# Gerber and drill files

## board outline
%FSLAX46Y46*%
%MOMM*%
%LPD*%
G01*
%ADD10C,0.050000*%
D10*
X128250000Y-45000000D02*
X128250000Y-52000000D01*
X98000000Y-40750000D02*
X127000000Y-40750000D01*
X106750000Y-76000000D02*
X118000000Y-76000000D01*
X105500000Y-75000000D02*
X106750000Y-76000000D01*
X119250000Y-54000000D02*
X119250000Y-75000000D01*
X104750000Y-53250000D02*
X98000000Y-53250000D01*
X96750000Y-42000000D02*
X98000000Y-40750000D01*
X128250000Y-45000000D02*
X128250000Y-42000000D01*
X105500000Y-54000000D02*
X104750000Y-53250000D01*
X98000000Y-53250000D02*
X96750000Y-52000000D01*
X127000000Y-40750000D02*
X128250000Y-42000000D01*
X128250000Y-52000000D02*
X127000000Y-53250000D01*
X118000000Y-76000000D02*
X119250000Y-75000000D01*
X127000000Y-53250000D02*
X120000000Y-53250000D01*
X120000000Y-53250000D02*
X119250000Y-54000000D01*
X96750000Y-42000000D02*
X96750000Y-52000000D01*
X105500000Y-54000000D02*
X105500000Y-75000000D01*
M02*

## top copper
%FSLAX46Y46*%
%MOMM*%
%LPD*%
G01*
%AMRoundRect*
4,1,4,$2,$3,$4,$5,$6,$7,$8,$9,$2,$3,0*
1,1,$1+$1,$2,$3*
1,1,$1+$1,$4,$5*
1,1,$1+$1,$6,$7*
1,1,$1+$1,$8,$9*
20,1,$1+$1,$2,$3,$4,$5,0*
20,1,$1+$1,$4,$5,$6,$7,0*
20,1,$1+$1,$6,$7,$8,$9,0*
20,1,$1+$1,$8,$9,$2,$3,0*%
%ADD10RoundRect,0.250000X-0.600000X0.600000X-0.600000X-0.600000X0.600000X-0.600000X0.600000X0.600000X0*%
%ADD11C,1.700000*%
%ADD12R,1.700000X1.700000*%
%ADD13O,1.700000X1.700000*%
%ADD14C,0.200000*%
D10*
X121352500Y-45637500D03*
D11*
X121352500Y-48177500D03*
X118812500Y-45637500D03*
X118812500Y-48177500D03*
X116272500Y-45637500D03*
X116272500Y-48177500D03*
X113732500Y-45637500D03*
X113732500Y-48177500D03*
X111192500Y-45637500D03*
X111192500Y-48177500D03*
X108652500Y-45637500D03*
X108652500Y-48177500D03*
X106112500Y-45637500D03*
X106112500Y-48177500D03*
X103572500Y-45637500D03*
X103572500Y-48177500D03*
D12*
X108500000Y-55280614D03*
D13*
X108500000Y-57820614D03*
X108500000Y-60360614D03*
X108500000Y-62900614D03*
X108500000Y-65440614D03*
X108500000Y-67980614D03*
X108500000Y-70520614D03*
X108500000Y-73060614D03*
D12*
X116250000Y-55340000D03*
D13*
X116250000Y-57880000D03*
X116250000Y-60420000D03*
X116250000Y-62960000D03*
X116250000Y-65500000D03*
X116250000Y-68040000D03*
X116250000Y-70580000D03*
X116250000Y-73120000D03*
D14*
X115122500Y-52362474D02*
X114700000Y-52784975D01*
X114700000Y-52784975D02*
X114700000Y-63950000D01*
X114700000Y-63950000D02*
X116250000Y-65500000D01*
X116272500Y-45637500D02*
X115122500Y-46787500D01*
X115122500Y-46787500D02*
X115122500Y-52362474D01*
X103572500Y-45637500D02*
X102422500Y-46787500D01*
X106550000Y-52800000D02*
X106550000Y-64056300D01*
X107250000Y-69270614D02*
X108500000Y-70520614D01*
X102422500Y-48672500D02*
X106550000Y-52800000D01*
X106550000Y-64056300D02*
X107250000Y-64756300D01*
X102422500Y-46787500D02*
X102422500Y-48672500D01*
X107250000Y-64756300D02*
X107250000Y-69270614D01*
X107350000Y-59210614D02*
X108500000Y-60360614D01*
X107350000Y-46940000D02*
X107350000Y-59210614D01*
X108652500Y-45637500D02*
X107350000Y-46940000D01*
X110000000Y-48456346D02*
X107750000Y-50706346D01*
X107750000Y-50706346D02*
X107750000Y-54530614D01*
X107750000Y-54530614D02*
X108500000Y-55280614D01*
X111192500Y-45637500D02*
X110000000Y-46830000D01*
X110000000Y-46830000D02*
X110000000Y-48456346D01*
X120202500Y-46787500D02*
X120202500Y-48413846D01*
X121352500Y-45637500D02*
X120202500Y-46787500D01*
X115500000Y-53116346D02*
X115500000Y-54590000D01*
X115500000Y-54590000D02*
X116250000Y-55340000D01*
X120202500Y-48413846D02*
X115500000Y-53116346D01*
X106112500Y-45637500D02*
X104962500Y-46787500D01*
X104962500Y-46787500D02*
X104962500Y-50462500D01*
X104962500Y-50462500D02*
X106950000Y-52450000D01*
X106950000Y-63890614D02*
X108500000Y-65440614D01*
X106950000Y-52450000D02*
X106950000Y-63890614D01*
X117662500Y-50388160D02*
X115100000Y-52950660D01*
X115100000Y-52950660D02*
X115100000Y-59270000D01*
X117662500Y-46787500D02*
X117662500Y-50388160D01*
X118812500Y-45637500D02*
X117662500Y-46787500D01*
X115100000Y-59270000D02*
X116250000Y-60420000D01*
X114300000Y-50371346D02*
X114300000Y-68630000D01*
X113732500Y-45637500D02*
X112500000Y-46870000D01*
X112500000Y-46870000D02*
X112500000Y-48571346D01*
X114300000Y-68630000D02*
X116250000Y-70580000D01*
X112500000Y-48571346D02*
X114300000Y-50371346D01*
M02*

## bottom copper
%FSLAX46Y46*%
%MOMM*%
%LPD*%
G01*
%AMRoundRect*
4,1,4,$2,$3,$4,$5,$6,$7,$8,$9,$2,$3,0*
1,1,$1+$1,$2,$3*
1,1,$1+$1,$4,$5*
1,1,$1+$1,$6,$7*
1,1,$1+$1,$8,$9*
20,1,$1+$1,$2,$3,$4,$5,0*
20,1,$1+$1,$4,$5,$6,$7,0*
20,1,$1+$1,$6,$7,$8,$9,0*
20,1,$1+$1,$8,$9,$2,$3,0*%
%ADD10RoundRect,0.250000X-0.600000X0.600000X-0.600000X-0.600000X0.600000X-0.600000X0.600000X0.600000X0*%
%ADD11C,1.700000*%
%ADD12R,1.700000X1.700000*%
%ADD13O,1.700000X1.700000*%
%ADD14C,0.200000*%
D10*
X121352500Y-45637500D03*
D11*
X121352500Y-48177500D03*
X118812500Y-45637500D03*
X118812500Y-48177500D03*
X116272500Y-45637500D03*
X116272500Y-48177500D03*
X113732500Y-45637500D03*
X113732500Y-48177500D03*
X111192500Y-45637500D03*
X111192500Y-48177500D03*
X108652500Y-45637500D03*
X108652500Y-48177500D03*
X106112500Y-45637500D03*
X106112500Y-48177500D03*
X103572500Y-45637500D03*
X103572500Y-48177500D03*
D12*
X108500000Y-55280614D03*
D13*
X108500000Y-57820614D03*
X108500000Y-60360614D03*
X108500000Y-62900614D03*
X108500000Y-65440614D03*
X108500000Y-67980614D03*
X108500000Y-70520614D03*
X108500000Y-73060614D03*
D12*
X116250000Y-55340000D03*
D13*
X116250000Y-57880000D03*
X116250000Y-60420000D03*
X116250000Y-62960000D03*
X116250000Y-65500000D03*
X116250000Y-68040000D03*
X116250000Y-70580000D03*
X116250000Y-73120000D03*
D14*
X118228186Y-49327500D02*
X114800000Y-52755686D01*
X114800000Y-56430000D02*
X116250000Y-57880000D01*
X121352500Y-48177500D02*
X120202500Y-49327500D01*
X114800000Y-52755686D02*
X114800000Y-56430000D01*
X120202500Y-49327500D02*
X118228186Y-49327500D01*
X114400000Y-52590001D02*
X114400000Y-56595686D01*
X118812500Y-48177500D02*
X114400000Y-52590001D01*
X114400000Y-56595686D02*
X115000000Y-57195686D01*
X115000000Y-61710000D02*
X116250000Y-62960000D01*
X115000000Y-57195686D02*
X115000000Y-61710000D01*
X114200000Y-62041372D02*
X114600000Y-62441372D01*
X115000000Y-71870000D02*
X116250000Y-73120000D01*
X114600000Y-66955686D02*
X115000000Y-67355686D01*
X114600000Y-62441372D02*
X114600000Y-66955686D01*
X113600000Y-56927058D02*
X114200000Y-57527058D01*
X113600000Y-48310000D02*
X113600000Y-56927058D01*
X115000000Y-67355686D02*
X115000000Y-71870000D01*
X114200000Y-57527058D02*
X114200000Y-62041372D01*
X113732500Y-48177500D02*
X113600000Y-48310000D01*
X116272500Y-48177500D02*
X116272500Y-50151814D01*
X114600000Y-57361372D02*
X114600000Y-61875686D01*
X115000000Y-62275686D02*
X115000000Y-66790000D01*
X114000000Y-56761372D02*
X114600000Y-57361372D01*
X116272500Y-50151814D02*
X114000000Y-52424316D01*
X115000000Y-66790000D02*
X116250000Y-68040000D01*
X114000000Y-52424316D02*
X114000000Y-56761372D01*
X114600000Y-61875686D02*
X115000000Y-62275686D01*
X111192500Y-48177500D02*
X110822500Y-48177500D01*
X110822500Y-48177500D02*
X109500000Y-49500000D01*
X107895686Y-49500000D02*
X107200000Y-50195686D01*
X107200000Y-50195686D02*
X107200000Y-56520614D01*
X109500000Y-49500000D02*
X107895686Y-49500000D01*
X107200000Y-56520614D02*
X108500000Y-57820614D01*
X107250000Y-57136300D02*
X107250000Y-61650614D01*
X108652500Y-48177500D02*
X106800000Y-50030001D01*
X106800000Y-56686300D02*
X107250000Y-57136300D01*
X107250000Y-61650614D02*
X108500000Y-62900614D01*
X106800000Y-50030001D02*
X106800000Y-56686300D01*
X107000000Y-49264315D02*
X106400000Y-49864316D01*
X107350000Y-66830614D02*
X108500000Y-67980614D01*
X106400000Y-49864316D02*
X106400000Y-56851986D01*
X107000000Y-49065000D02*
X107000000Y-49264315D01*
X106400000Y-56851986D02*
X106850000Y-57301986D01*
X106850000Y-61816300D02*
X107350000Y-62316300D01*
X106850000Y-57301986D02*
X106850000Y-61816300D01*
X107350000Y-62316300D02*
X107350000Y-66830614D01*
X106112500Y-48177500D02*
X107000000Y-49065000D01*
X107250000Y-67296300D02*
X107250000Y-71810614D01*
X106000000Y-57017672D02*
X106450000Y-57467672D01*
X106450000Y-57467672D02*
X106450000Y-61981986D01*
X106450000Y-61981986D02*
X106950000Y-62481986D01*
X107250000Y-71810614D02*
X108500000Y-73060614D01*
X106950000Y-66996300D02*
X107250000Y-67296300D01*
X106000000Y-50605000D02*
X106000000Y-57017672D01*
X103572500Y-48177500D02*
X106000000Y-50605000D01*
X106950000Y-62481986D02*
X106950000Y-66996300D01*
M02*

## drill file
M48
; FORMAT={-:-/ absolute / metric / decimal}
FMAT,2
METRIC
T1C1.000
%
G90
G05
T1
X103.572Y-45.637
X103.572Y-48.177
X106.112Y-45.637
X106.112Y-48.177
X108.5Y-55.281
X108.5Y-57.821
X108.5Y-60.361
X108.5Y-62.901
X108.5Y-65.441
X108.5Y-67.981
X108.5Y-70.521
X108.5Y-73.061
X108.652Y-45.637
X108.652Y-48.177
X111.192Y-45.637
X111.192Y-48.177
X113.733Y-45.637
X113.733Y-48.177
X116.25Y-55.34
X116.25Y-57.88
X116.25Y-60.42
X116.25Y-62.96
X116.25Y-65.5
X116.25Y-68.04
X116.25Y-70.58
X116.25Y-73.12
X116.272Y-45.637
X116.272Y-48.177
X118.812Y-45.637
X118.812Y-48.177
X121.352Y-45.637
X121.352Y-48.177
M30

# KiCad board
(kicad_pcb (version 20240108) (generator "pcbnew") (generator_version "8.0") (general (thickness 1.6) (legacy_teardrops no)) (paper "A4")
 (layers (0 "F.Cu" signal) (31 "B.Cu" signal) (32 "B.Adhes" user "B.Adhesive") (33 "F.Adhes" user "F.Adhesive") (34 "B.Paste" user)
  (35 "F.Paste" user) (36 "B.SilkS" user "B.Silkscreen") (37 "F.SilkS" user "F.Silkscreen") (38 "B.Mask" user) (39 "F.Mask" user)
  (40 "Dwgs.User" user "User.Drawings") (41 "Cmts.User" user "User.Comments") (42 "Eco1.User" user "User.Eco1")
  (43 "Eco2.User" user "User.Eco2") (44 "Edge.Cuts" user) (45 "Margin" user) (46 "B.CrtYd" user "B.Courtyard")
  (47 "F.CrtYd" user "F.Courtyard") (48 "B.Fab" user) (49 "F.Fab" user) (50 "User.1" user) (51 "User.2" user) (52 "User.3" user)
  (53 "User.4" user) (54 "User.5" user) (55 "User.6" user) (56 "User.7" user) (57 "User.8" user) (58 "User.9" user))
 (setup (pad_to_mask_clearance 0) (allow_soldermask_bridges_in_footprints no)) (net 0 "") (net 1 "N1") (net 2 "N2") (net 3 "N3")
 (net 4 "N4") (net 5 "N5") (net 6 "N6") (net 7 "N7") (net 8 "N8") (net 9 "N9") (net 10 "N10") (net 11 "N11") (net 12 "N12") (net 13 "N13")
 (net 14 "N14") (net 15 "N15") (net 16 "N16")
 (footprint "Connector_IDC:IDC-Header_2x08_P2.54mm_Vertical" (layer "F.Cu") (at 121.3525 45.6375 -90)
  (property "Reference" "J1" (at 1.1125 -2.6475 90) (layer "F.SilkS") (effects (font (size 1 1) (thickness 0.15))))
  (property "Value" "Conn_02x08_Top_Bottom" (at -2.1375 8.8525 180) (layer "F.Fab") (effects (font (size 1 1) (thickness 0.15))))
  (pad "1" thru_hole roundrect (at 0 0 270) (size 1.7 1.7) (drill 1) (layers "*.Cu" "*.Mask") (remove_unused_layers no)
   (roundrect_rratio 0.147059) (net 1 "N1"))
  (pad "2" thru_hole circle (at 2.54 0 270) (size 1.7 1.7) (drill 1) (layers "*.Cu" "*.Mask") (remove_unused_layers no) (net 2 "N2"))
  (pad "3" thru_hole circle (at 0 2.54 270) (size 1.7 1.7) (drill 1) (layers "*.Cu" "*.Mask") (remove_unused_layers no) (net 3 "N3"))
  (pad "4" thru_hole circle (at 2.54 2.54 270) (size 1.7 1.7) (drill 1) (layers "*.Cu" "*.Mask") (remove_unused_layers no) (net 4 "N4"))
  (pad "5" thru_hole circle (at 0 5.08 270) (size 1.7 1.7) (drill 1) (layers "*.Cu" "*.Mask") (remove_unused_layers no) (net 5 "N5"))
  (pad "6" thru_hole circle (at 2.54 5.08 270) (size 1.7 1.7) (drill 1) (layers "*.Cu" "*.Mask") (remove_unused_layers no) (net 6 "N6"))
  (pad "7" thru_hole circle (at 0 7.62 270) (size 1.7 1.7) (drill 1) (layers "*.Cu" "*.Mask") (remove_unused_layers no) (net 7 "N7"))
  (pad "8" thru_hole circle (at 2.54 7.62 270) (size 1.7 1.7) (drill 1) (layers "*.Cu" "*.Mask") (remove_unused_layers no) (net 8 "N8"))
  (pad "9" thru_hole circle (at 0 10.16 270) (size 1.7 1.7) (drill 1) (layers "*.Cu" "*.Mask") (remove_unused_layers no) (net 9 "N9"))
  (pad "10" thru_hole circle (at 2.54 10.16 270) (size 1.7 1.7) (drill 1) (layers "*.Cu" "*.Mask") (remove_unused_layers no) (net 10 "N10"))
  (pad "11" thru_hole circle (at 0 12.7 270) (size 1.7 1.7) (drill 1) (layers "*.Cu" "*.Mask") (remove_unused_layers no) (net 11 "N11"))
  (pad "12" thru_hole circle (at 2.54 12.7 270) (size 1.7 1.7) (drill 1) (layers "*.Cu" "*.Mask") (remove_unused_layers no) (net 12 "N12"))
  (pad "13" thru_hole circle (at 0 15.24 270) (size 1.7 1.7) (drill 1) (layers "*.Cu" "*.Mask") (remove_unused_layers no) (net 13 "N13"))
  (pad "14" thru_hole circle (at 2.54 15.24 270) (size 1.7 1.7) (drill 1) (layers "*.Cu" "*.Mask") (remove_unused_layers no) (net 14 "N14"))
  (pad "15" thru_hole circle (at 0 17.78 270) (size 1.7 1.7) (drill 1) (layers "*.Cu" "*.Mask") (remove_unused_layers no) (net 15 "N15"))
  (pad "16" thru_hole circle (at 2.54 17.78 270) (size 1.7 1.7) (drill 1) (layers "*.Cu" "*.Mask") (remove_unused_layers no) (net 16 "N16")))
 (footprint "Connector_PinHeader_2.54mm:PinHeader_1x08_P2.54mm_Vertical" (layer "B.Cu") (at 108.5 55.280614 180)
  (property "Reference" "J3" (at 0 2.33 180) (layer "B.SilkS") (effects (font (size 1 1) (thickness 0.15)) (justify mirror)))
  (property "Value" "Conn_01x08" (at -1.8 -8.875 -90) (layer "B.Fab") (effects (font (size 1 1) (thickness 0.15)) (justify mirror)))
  (pad "1" thru_hole rect (at 0 0 180) (size 1.7 1.7) (drill 1) (layers "*.Cu" "*.Mask") (remove_unused_layers no) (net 9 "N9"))
  (pad "2" thru_hole oval (at 0 -2.54 180) (size 1.7 1.7) (drill 1) (layers "*.Cu" "*.Mask") (remove_unused_layers no) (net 10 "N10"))
  (pad "3" thru_hole oval (at 0 -5.08 180) (size 1.7 1.7) (drill 1) (layers "*.Cu" "*.Mask") (remove_unused_layers no) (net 11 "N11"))
  (pad "4" thru_hole oval (at 0 -7.62 180) (size 1.7 1.7) (drill 1) (layers "*.Cu" "*.Mask") (remove_unused_layers no) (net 12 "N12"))
  (pad "5" thru_hole oval (at 0 -10.16 180) (size 1.7 1.7) (drill 1) (layers "*.Cu" "*.Mask") (remove_unused_layers no) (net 13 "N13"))
  (pad "6" thru_hole oval (at 0 -12.7 180) (size 1.7 1.7) (drill 1) (layers "*.Cu" "*.Mask") (remove_unused_layers no) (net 14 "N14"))
  (pad "7" thru_hole oval (at 0 -15.24 180) (size 1.7 1.7) (drill 1) (layers "*.Cu" "*.Mask") (remove_unused_layers no) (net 15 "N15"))
  (pad "8" thru_hole oval (at 0 -17.78 180) (size 1.7 1.7) (drill 1) (layers "*.Cu" "*.Mask") (remove_unused_layers no) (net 16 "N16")))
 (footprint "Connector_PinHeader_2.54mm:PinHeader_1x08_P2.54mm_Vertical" (layer "B.Cu") (at 116.25 55.34 180)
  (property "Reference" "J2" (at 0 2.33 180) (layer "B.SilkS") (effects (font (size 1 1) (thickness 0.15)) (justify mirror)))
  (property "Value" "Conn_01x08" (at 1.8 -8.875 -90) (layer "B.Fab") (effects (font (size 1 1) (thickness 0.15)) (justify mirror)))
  (pad "1" thru_hole rect (at 0 0 180) (size 1.7 1.7) (drill 1) (layers "*.Cu" "*.Mask") (remove_unused_layers no) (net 1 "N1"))
  (pad "2" thru_hole oval (at 0 -2.54 180) (size 1.7 1.7) (drill 1) (layers "*.Cu" "*.Mask") (remove_unused_layers no) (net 2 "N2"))
  (pad "3" thru_hole oval (at 0 -5.08 180) (size 1.7 1.7) (drill 1) (layers "*.Cu" "*.Mask") (remove_unused_layers no) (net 3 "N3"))
  (pad "4" thru_hole oval (at 0 -7.62 180) (size 1.7 1.7) (drill 1) (layers "*.Cu" "*.Mask") (remove_unused_layers no) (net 4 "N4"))
  (pad "5" thru_hole oval (at 0 -10.16 180) (size 1.7 1.7) (drill 1) (layers "*.Cu" "*.Mask") (remove_unused_layers no) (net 5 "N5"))
  (pad "6" thru_hole oval (at 0 -12.7 180) (size 1.7 1.7) (drill 1) (layers "*.Cu" "*.Mask") (remove_unused_layers no) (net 6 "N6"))
  (pad "7" thru_hole oval (at 0 -15.24 180) (size 1.7 1.7) (drill 1) (layers "*.Cu" "*.Mask") (remove_unused_layers no) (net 7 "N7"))
  (pad "8" thru_hole oval (at 0 -17.78 180) (size 1.7 1.7) (drill 1) (layers "*.Cu" "*.Mask") (remove_unused_layers no) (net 8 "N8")))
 (gr_line (start 128.25 45) (end 128.25 52) (stroke (width 0.05) (type default)) (layer "Edge.Cuts"))
 (gr_line (start 98 40.75) (end 127 40.75) (stroke (width 0.05) (type default)) (layer "Edge.Cuts"))
 (gr_line (start 106.75 76) (end 118 76) (stroke (width 0.05) (type default)) (layer "Edge.Cuts"))
 (gr_line (start 105.5 75) (end 106.75 76) (stroke (width 0.05) (type default)) (layer "Edge.Cuts"))
 (gr_line (start 119.25 54) (end 119.25 75) (stroke (width 0.05) (type default)) (layer "Edge.Cuts"))
 (gr_line (start 104.75 53.25) (end 98 53.25) (stroke (width 0.05) (type default)) (layer "Edge.Cuts"))
 (gr_line (start 96.75 42) (end 98 40.75) (stroke (width 0.05) (type default)) (layer "Edge.Cuts"))
 (gr_line (start 128.25 45) (end 128.25 42) (stroke (width 0.05) (type default)) (layer "Edge.Cuts"))
 (gr_line (start 105.5 54) (end 104.75 53.25) (stroke (width 0.05) (type default)) (layer "Edge.Cuts"))
 (gr_line (start 98 53.25) (end 96.75 52) (stroke (width 0.05) (type default)) (layer "Edge.Cuts"))
 (gr_line (start 127 40.75) (end 128.25 42) (stroke (width 0.05) (type default)) (layer "Edge.Cuts"))
 (gr_line (start 128.25 52) (end 127 53.25) (stroke (width 0.05) (type default)) (layer "Edge.Cuts"))
 (gr_line (start 118 76) (end 119.25 75) (stroke (width 0.05) (type default)) (layer "Edge.Cuts"))
 (gr_line (start 127 53.25) (end 120 53.25) (stroke (width 0.05) (type default)) (layer "Edge.Cuts"))
 (gr_line (start 120 53.25) (end 119.25 54) (stroke (width 0.05) (type default)) (layer "Edge.Cuts"))
 (gr_line (start 96.75 42) (end 96.75 52) (stroke (width 0.05) (type default)) (layer "Edge.Cuts"))
 (gr_line (start 105.5 54) (end 105.5 75) (stroke (width 0.05) (type default)) (layer "Edge.Cuts"))
 (segment (start 115.1225 52.362474) (end 114.7 52.784975) (width 0.2) (layer "F.Cu") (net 5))
 (segment (start 114.7 52.784975) (end 114.7 63.95) (width 0.2) (layer "F.Cu") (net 5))
 (segment (start 114.7 63.95) (end 116.25 65.5) (width 0.2) (layer "F.Cu") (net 5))
 (segment (start 116.2725 45.6375) (end 115.1225 46.7875) (width 0.2) (layer "F.Cu") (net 5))
 (segment (start 115.1225 46.7875) (end 115.1225 52.362474) (width 0.2) (layer "F.Cu") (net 5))
 (segment (start 103.5725 45.6375) (end 102.4225 46.7875) (width 0.2) (layer "F.Cu") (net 15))
 (segment (start 106.55 52.8) (end 106.55 64.0563) (width 0.2) (layer "F.Cu") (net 15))
 (segment (start 107.25 69.270614) (end 108.5 70.520614) (width 0.2) (layer "F.Cu") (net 15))
 (segment (start 102.4225 48.6725) (end 106.55 52.8) (width 0.2) (layer "F.Cu") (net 15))
 (segment (start 106.55 64.0563) (end 107.25 64.7563) (width 0.2) (layer "F.Cu") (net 15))
 (segment (start 102.4225 46.7875) (end 102.4225 48.6725) (width 0.2) (layer "F.Cu") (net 15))
 (segment (start 107.25 64.7563) (end 107.25 69.270614) (width 0.2) (layer "F.Cu") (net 15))
 (segment (start 118.228186 49.3275) (end 114.8 52.755686) (width 0.2) (layer "B.Cu") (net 2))
 (segment (start 114.8 56.43) (end 116.25 57.88) (width 0.2) (layer "B.Cu") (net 2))
 (segment (start 121.3525 48.1775) (end 120.2025 49.3275) (width 0.2) (layer "B.Cu") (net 2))
 (segment (start 114.8 52.755686) (end 114.8 56.43) (width 0.2) (layer "B.Cu") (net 2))
 (segment (start 120.2025 49.3275) (end 118.228186 49.3275) (width 0.2) (layer "B.Cu") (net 2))
 (segment (start 114.4 52.590001) (end 114.4 56.595686) (width 0.2) (layer "B.Cu") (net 4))
 (segment (start 118.8125 48.1775) (end 114.4 52.590001) (width 0.2) (layer "B.Cu") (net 4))
 (segment (start 114.4 56.595686) (end 115 57.195686) (width 0.2) (layer "B.Cu") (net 4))
 (segment (start 115 61.71) (end 116.25 62.96) (width 0.2) (layer "B.Cu") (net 4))
 (segment (start 115 57.195686) (end 115 61.71) (width 0.2) (layer "B.Cu") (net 4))
 (segment (start 114.2 62.041372) (end 114.6 62.441372) (width 0.2) (layer "B.Cu") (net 8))
 (segment (start 115 71.87) (end 116.25 73.12) (width 0.2) (layer "B.Cu") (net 8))
 (segment (start 114.6 66.955686) (end 115 67.355686) (width 0.2) (layer "B.Cu") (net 8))
 (segment (start 114.6 62.441372) (end 114.6 66.955686) (width 0.2) (layer "B.Cu") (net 8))
 (segment (start 113.6 56.927058) (end 114.2 57.527058) (width 0.2) (layer "B.Cu") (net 8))
 (segment (start 113.6 48.31) (end 113.6 56.927058) (width 0.2) (layer "B.Cu") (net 8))
 (segment (start 115 67.355686) (end 115 71.87) (width 0.2) (layer "B.Cu") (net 8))
 (segment (start 114.2 57.527058) (end 114.2 62.041372) (width 0.2) (layer "B.Cu") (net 8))
 (segment (start 113.7325 48.1775) (end 113.6 48.31) (width 0.2) (layer "B.Cu") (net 8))
 (segment (start 116.2725 48.1775) (end 116.2725 50.151814) (width 0.2) (layer "B.Cu") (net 6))
 (segment (start 114.6 57.361372) (end 114.6 61.875686) (width 0.2) (layer "B.Cu") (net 6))
 (segment (start 115 62.275686) (end 115 66.79) (width 0.2) (layer "B.Cu") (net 6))
 (segment (start 114 56.761372) (end 114.6 57.361372) (width 0.2) (layer "B.Cu") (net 6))
 (segment (start 116.2725 50.151814) (end 114 52.424316) (width 0.2) (layer "B.Cu") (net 6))
 (segment (start 115 66.79) (end 116.25 68.04) (width 0.2) (layer "B.Cu") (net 6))
 (segment (start 114 52.424316) (end 114 56.761372) (width 0.2) (layer "B.Cu") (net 6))
 (segment (start 114.6 61.875686) (end 115 62.275686) (width 0.2) (layer "B.Cu") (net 6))
 (segment (start 107.35 59.210614) (end 108.5 60.360614) (width 0.2) (layer "F.Cu") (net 11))
 (segment (start 107.35 46.94) (end 107.35 59.210614) (width 0.2) (layer "F.Cu") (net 11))
 (segment (start 108.6525 45.6375) (end 107.35 46.94) (width 0.2) (layer "F.Cu") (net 11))
 (segment (start 110 48.456346) (end 107.75 50.706346) (width 0.2) (layer "F.Cu") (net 9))
 (segment (start 107.75 50.706346) (end 107.75 54.530614) (width 0.2) (layer "F.Cu") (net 9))
 (segment (start 107.75 54.530614) (end 108.5 55.280614) (width 0.2) (layer "F.Cu") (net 9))
 (segment (start 111.1925 45.6375) (end 110 46.83) (width 0.2) (layer "F.Cu") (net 9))
 (segment (start 110 46.83) (end 110 48.456346) (width 0.2) (layer "F.Cu") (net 9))
 (segment (start 111.1925 48.1775) (end 110.8225 48.1775) (width 0.2) (layer "B.Cu") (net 10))
 (segment (start 110.8225 48.1775) (end 109.5 49.5) (width 0.2) (layer "B.Cu") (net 10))
 (segment (start 107.895686 49.5) (end 107.2 50.195686) (width 0.2) (layer "B.Cu") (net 10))
 (segment (start 107.2 50.195686) (end 107.2 56.520614) (width 0.2) (layer "B.Cu") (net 10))
 (segment (start 109.5 49.5) (end 107.895686 49.5) (width 0.2) (layer "B.Cu") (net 10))
 (segment (start 107.2 56.520614) (end 108.5 57.820614) (width 0.2) (layer "B.Cu") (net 10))
 (segment (start 107.25 57.1363) (end 107.25 61.650614) (width 0.2) (layer "B.Cu") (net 12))
 (segment (start 108.6525 48.1775) (end 106.8 50.030001) (width 0.2) (layer "B.Cu") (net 12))
 (segment (start 106.8 56.6863) (end 107.25 57.1363) (width 0.2) (layer "B.Cu") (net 12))
 (segment (start 107.25 61.650614) (end 108.5 62.900614) (width 0.2) (layer "B.Cu") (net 12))
 (segment (start 106.8 50.030001) (end 106.8 56.6863) (width 0.2) (layer "B.Cu") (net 12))
 (segment (start 120.2025 46.7875) (end 120.2025 48.413846) (width 0.2) (layer "F.Cu") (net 1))
 (segment (start 121.3525 45.6375) (end 120.2025 46.7875) (width 0.2) (layer "F.Cu") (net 1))
 (segment (start 115.5 53.116346) (end 115.5 54.59) (width 0.2) (layer "F.Cu") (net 1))
 (segment (start 115.5 54.59) (end 116.25 55.34) (width 0.2) (layer "F.Cu") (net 1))
 (segment (start 120.2025 48.413846) (end 115.5 53.116346) (width 0.2) (layer "F.Cu") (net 1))
 (segment (start 106.1125 45.6375) (end 104.9625 46.7875) (width 0.2) (layer "F.Cu") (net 13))
 (segment (start 104.9625 46.7875) (end 104.9625 50.4625) (width 0.2) (layer "F.Cu") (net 13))
 (segment (start 104.9625 50.4625) (end 106.95 52.45) (width 0.2) (layer "F.Cu") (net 13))
 (segment (start 106.95 63.890614) (end 108.5 65.440614) (width 0.2) (layer "F.Cu") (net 13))
 (segment (start 106.95 52.45) (end 106.95 63.890614) (width 0.2) (layer "F.Cu") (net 13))
 (segment (start 117.6625 50.38816) (end 115.1 52.95066) (width 0.2) (layer "F.Cu") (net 3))
 (segment (start 115.1 52.95066) (end 115.1 59.27) (width 0.2) (layer "F.Cu") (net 3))
 (segment (start 117.6625 46.7875) (end 117.6625 50.38816) (width 0.2) (layer "F.Cu") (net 3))
 (segment (start 118.8125 45.6375) (end 117.6625 46.7875) (width 0.2) (layer "F.Cu") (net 3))
 (segment (start 115.1 59.27) (end 116.25 60.42) (width 0.2) (layer "F.Cu") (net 3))
 (segment (start 107 49.264315) (end 106.4 49.864316) (width 0.2) (layer "B.Cu") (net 14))
 (segment (start 107.35 66.830614) (end 108.5 67.980614) (width 0.2) (layer "B.Cu") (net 14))
 (segment (start 106.4 49.864316) (end 106.4 56.851986) (width 0.2) (layer "B.Cu") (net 14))
 (segment (start 107 49.065) (end 107 49.264315) (width 0.2) (layer "B.Cu") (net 14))
 (segment (start 106.4 56.851986) (end 106.85 57.301986) (width 0.2) (layer "B.Cu") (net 14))
 (segment (start 106.85 61.8163) (end 107.35 62.3163) (width 0.2) (layer "B.Cu") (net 14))
 (segment (start 106.85 57.301986) (end 106.85 61.8163) (width 0.2) (layer "B.Cu") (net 14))
 (segment (start 107.35 62.3163) (end 107.35 66.830614) (width 0.2) (layer "B.Cu") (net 14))
 (segment (start 106.1125 48.1775) (end 107 49.065) (width 0.2) (layer "B.Cu") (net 14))
 (segment (start 107.25 67.2963) (end 107.25 71.810614) (width 0.2) (layer "B.Cu") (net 16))
 (segment (start 106 57.017672) (end 106.45 57.467672) (width 0.2) (layer "B.Cu") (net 16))
 (segment (start 106.45 57.467672) (end 106.45 61.981986) (width 0.2) (layer "B.Cu") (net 16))
 (segment (start 106.45 61.981986) (end 106.95 62.481986) (width 0.2) (layer "B.Cu") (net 16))
 (segment (start 107.25 71.810614) (end 108.5 73.060614) (width 0.2) (layer "B.Cu") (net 16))
 (segment (start 106.95 66.9963) (end 107.25 67.2963) (width 0.2) (layer "B.Cu") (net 16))
 (segment (start 106 50.605) (end 106 57.017672) (width 0.2) (layer "B.Cu") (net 16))
 (segment (start 103.5725 48.1775) (end 106 50.605) (width 0.2) (layer "B.Cu") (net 16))
 (segment (start 106.95 62.481986) (end 106.95 66.9963) (width 0.2) (layer "B.Cu") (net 16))
 (segment (start 114.3 50.371346) (end 114.3 68.63) (width 0.2) (layer "F.Cu") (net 7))
 (segment (start 113.7325 45.6375) (end 112.5 46.87) (width 0.2) (layer "F.Cu") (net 7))
 (segment (start 112.5 46.87) (end 112.5 48.571346) (width 0.2) (layer "F.Cu") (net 7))
 (segment (start 114.3 68.63) (end 116.25 70.58) (width 0.2) (layer "F.Cu") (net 7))
 (segment (start 112.5 48.571346) (end 114.3 50.371346) (width 0.2) (layer "F.Cu") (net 7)))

